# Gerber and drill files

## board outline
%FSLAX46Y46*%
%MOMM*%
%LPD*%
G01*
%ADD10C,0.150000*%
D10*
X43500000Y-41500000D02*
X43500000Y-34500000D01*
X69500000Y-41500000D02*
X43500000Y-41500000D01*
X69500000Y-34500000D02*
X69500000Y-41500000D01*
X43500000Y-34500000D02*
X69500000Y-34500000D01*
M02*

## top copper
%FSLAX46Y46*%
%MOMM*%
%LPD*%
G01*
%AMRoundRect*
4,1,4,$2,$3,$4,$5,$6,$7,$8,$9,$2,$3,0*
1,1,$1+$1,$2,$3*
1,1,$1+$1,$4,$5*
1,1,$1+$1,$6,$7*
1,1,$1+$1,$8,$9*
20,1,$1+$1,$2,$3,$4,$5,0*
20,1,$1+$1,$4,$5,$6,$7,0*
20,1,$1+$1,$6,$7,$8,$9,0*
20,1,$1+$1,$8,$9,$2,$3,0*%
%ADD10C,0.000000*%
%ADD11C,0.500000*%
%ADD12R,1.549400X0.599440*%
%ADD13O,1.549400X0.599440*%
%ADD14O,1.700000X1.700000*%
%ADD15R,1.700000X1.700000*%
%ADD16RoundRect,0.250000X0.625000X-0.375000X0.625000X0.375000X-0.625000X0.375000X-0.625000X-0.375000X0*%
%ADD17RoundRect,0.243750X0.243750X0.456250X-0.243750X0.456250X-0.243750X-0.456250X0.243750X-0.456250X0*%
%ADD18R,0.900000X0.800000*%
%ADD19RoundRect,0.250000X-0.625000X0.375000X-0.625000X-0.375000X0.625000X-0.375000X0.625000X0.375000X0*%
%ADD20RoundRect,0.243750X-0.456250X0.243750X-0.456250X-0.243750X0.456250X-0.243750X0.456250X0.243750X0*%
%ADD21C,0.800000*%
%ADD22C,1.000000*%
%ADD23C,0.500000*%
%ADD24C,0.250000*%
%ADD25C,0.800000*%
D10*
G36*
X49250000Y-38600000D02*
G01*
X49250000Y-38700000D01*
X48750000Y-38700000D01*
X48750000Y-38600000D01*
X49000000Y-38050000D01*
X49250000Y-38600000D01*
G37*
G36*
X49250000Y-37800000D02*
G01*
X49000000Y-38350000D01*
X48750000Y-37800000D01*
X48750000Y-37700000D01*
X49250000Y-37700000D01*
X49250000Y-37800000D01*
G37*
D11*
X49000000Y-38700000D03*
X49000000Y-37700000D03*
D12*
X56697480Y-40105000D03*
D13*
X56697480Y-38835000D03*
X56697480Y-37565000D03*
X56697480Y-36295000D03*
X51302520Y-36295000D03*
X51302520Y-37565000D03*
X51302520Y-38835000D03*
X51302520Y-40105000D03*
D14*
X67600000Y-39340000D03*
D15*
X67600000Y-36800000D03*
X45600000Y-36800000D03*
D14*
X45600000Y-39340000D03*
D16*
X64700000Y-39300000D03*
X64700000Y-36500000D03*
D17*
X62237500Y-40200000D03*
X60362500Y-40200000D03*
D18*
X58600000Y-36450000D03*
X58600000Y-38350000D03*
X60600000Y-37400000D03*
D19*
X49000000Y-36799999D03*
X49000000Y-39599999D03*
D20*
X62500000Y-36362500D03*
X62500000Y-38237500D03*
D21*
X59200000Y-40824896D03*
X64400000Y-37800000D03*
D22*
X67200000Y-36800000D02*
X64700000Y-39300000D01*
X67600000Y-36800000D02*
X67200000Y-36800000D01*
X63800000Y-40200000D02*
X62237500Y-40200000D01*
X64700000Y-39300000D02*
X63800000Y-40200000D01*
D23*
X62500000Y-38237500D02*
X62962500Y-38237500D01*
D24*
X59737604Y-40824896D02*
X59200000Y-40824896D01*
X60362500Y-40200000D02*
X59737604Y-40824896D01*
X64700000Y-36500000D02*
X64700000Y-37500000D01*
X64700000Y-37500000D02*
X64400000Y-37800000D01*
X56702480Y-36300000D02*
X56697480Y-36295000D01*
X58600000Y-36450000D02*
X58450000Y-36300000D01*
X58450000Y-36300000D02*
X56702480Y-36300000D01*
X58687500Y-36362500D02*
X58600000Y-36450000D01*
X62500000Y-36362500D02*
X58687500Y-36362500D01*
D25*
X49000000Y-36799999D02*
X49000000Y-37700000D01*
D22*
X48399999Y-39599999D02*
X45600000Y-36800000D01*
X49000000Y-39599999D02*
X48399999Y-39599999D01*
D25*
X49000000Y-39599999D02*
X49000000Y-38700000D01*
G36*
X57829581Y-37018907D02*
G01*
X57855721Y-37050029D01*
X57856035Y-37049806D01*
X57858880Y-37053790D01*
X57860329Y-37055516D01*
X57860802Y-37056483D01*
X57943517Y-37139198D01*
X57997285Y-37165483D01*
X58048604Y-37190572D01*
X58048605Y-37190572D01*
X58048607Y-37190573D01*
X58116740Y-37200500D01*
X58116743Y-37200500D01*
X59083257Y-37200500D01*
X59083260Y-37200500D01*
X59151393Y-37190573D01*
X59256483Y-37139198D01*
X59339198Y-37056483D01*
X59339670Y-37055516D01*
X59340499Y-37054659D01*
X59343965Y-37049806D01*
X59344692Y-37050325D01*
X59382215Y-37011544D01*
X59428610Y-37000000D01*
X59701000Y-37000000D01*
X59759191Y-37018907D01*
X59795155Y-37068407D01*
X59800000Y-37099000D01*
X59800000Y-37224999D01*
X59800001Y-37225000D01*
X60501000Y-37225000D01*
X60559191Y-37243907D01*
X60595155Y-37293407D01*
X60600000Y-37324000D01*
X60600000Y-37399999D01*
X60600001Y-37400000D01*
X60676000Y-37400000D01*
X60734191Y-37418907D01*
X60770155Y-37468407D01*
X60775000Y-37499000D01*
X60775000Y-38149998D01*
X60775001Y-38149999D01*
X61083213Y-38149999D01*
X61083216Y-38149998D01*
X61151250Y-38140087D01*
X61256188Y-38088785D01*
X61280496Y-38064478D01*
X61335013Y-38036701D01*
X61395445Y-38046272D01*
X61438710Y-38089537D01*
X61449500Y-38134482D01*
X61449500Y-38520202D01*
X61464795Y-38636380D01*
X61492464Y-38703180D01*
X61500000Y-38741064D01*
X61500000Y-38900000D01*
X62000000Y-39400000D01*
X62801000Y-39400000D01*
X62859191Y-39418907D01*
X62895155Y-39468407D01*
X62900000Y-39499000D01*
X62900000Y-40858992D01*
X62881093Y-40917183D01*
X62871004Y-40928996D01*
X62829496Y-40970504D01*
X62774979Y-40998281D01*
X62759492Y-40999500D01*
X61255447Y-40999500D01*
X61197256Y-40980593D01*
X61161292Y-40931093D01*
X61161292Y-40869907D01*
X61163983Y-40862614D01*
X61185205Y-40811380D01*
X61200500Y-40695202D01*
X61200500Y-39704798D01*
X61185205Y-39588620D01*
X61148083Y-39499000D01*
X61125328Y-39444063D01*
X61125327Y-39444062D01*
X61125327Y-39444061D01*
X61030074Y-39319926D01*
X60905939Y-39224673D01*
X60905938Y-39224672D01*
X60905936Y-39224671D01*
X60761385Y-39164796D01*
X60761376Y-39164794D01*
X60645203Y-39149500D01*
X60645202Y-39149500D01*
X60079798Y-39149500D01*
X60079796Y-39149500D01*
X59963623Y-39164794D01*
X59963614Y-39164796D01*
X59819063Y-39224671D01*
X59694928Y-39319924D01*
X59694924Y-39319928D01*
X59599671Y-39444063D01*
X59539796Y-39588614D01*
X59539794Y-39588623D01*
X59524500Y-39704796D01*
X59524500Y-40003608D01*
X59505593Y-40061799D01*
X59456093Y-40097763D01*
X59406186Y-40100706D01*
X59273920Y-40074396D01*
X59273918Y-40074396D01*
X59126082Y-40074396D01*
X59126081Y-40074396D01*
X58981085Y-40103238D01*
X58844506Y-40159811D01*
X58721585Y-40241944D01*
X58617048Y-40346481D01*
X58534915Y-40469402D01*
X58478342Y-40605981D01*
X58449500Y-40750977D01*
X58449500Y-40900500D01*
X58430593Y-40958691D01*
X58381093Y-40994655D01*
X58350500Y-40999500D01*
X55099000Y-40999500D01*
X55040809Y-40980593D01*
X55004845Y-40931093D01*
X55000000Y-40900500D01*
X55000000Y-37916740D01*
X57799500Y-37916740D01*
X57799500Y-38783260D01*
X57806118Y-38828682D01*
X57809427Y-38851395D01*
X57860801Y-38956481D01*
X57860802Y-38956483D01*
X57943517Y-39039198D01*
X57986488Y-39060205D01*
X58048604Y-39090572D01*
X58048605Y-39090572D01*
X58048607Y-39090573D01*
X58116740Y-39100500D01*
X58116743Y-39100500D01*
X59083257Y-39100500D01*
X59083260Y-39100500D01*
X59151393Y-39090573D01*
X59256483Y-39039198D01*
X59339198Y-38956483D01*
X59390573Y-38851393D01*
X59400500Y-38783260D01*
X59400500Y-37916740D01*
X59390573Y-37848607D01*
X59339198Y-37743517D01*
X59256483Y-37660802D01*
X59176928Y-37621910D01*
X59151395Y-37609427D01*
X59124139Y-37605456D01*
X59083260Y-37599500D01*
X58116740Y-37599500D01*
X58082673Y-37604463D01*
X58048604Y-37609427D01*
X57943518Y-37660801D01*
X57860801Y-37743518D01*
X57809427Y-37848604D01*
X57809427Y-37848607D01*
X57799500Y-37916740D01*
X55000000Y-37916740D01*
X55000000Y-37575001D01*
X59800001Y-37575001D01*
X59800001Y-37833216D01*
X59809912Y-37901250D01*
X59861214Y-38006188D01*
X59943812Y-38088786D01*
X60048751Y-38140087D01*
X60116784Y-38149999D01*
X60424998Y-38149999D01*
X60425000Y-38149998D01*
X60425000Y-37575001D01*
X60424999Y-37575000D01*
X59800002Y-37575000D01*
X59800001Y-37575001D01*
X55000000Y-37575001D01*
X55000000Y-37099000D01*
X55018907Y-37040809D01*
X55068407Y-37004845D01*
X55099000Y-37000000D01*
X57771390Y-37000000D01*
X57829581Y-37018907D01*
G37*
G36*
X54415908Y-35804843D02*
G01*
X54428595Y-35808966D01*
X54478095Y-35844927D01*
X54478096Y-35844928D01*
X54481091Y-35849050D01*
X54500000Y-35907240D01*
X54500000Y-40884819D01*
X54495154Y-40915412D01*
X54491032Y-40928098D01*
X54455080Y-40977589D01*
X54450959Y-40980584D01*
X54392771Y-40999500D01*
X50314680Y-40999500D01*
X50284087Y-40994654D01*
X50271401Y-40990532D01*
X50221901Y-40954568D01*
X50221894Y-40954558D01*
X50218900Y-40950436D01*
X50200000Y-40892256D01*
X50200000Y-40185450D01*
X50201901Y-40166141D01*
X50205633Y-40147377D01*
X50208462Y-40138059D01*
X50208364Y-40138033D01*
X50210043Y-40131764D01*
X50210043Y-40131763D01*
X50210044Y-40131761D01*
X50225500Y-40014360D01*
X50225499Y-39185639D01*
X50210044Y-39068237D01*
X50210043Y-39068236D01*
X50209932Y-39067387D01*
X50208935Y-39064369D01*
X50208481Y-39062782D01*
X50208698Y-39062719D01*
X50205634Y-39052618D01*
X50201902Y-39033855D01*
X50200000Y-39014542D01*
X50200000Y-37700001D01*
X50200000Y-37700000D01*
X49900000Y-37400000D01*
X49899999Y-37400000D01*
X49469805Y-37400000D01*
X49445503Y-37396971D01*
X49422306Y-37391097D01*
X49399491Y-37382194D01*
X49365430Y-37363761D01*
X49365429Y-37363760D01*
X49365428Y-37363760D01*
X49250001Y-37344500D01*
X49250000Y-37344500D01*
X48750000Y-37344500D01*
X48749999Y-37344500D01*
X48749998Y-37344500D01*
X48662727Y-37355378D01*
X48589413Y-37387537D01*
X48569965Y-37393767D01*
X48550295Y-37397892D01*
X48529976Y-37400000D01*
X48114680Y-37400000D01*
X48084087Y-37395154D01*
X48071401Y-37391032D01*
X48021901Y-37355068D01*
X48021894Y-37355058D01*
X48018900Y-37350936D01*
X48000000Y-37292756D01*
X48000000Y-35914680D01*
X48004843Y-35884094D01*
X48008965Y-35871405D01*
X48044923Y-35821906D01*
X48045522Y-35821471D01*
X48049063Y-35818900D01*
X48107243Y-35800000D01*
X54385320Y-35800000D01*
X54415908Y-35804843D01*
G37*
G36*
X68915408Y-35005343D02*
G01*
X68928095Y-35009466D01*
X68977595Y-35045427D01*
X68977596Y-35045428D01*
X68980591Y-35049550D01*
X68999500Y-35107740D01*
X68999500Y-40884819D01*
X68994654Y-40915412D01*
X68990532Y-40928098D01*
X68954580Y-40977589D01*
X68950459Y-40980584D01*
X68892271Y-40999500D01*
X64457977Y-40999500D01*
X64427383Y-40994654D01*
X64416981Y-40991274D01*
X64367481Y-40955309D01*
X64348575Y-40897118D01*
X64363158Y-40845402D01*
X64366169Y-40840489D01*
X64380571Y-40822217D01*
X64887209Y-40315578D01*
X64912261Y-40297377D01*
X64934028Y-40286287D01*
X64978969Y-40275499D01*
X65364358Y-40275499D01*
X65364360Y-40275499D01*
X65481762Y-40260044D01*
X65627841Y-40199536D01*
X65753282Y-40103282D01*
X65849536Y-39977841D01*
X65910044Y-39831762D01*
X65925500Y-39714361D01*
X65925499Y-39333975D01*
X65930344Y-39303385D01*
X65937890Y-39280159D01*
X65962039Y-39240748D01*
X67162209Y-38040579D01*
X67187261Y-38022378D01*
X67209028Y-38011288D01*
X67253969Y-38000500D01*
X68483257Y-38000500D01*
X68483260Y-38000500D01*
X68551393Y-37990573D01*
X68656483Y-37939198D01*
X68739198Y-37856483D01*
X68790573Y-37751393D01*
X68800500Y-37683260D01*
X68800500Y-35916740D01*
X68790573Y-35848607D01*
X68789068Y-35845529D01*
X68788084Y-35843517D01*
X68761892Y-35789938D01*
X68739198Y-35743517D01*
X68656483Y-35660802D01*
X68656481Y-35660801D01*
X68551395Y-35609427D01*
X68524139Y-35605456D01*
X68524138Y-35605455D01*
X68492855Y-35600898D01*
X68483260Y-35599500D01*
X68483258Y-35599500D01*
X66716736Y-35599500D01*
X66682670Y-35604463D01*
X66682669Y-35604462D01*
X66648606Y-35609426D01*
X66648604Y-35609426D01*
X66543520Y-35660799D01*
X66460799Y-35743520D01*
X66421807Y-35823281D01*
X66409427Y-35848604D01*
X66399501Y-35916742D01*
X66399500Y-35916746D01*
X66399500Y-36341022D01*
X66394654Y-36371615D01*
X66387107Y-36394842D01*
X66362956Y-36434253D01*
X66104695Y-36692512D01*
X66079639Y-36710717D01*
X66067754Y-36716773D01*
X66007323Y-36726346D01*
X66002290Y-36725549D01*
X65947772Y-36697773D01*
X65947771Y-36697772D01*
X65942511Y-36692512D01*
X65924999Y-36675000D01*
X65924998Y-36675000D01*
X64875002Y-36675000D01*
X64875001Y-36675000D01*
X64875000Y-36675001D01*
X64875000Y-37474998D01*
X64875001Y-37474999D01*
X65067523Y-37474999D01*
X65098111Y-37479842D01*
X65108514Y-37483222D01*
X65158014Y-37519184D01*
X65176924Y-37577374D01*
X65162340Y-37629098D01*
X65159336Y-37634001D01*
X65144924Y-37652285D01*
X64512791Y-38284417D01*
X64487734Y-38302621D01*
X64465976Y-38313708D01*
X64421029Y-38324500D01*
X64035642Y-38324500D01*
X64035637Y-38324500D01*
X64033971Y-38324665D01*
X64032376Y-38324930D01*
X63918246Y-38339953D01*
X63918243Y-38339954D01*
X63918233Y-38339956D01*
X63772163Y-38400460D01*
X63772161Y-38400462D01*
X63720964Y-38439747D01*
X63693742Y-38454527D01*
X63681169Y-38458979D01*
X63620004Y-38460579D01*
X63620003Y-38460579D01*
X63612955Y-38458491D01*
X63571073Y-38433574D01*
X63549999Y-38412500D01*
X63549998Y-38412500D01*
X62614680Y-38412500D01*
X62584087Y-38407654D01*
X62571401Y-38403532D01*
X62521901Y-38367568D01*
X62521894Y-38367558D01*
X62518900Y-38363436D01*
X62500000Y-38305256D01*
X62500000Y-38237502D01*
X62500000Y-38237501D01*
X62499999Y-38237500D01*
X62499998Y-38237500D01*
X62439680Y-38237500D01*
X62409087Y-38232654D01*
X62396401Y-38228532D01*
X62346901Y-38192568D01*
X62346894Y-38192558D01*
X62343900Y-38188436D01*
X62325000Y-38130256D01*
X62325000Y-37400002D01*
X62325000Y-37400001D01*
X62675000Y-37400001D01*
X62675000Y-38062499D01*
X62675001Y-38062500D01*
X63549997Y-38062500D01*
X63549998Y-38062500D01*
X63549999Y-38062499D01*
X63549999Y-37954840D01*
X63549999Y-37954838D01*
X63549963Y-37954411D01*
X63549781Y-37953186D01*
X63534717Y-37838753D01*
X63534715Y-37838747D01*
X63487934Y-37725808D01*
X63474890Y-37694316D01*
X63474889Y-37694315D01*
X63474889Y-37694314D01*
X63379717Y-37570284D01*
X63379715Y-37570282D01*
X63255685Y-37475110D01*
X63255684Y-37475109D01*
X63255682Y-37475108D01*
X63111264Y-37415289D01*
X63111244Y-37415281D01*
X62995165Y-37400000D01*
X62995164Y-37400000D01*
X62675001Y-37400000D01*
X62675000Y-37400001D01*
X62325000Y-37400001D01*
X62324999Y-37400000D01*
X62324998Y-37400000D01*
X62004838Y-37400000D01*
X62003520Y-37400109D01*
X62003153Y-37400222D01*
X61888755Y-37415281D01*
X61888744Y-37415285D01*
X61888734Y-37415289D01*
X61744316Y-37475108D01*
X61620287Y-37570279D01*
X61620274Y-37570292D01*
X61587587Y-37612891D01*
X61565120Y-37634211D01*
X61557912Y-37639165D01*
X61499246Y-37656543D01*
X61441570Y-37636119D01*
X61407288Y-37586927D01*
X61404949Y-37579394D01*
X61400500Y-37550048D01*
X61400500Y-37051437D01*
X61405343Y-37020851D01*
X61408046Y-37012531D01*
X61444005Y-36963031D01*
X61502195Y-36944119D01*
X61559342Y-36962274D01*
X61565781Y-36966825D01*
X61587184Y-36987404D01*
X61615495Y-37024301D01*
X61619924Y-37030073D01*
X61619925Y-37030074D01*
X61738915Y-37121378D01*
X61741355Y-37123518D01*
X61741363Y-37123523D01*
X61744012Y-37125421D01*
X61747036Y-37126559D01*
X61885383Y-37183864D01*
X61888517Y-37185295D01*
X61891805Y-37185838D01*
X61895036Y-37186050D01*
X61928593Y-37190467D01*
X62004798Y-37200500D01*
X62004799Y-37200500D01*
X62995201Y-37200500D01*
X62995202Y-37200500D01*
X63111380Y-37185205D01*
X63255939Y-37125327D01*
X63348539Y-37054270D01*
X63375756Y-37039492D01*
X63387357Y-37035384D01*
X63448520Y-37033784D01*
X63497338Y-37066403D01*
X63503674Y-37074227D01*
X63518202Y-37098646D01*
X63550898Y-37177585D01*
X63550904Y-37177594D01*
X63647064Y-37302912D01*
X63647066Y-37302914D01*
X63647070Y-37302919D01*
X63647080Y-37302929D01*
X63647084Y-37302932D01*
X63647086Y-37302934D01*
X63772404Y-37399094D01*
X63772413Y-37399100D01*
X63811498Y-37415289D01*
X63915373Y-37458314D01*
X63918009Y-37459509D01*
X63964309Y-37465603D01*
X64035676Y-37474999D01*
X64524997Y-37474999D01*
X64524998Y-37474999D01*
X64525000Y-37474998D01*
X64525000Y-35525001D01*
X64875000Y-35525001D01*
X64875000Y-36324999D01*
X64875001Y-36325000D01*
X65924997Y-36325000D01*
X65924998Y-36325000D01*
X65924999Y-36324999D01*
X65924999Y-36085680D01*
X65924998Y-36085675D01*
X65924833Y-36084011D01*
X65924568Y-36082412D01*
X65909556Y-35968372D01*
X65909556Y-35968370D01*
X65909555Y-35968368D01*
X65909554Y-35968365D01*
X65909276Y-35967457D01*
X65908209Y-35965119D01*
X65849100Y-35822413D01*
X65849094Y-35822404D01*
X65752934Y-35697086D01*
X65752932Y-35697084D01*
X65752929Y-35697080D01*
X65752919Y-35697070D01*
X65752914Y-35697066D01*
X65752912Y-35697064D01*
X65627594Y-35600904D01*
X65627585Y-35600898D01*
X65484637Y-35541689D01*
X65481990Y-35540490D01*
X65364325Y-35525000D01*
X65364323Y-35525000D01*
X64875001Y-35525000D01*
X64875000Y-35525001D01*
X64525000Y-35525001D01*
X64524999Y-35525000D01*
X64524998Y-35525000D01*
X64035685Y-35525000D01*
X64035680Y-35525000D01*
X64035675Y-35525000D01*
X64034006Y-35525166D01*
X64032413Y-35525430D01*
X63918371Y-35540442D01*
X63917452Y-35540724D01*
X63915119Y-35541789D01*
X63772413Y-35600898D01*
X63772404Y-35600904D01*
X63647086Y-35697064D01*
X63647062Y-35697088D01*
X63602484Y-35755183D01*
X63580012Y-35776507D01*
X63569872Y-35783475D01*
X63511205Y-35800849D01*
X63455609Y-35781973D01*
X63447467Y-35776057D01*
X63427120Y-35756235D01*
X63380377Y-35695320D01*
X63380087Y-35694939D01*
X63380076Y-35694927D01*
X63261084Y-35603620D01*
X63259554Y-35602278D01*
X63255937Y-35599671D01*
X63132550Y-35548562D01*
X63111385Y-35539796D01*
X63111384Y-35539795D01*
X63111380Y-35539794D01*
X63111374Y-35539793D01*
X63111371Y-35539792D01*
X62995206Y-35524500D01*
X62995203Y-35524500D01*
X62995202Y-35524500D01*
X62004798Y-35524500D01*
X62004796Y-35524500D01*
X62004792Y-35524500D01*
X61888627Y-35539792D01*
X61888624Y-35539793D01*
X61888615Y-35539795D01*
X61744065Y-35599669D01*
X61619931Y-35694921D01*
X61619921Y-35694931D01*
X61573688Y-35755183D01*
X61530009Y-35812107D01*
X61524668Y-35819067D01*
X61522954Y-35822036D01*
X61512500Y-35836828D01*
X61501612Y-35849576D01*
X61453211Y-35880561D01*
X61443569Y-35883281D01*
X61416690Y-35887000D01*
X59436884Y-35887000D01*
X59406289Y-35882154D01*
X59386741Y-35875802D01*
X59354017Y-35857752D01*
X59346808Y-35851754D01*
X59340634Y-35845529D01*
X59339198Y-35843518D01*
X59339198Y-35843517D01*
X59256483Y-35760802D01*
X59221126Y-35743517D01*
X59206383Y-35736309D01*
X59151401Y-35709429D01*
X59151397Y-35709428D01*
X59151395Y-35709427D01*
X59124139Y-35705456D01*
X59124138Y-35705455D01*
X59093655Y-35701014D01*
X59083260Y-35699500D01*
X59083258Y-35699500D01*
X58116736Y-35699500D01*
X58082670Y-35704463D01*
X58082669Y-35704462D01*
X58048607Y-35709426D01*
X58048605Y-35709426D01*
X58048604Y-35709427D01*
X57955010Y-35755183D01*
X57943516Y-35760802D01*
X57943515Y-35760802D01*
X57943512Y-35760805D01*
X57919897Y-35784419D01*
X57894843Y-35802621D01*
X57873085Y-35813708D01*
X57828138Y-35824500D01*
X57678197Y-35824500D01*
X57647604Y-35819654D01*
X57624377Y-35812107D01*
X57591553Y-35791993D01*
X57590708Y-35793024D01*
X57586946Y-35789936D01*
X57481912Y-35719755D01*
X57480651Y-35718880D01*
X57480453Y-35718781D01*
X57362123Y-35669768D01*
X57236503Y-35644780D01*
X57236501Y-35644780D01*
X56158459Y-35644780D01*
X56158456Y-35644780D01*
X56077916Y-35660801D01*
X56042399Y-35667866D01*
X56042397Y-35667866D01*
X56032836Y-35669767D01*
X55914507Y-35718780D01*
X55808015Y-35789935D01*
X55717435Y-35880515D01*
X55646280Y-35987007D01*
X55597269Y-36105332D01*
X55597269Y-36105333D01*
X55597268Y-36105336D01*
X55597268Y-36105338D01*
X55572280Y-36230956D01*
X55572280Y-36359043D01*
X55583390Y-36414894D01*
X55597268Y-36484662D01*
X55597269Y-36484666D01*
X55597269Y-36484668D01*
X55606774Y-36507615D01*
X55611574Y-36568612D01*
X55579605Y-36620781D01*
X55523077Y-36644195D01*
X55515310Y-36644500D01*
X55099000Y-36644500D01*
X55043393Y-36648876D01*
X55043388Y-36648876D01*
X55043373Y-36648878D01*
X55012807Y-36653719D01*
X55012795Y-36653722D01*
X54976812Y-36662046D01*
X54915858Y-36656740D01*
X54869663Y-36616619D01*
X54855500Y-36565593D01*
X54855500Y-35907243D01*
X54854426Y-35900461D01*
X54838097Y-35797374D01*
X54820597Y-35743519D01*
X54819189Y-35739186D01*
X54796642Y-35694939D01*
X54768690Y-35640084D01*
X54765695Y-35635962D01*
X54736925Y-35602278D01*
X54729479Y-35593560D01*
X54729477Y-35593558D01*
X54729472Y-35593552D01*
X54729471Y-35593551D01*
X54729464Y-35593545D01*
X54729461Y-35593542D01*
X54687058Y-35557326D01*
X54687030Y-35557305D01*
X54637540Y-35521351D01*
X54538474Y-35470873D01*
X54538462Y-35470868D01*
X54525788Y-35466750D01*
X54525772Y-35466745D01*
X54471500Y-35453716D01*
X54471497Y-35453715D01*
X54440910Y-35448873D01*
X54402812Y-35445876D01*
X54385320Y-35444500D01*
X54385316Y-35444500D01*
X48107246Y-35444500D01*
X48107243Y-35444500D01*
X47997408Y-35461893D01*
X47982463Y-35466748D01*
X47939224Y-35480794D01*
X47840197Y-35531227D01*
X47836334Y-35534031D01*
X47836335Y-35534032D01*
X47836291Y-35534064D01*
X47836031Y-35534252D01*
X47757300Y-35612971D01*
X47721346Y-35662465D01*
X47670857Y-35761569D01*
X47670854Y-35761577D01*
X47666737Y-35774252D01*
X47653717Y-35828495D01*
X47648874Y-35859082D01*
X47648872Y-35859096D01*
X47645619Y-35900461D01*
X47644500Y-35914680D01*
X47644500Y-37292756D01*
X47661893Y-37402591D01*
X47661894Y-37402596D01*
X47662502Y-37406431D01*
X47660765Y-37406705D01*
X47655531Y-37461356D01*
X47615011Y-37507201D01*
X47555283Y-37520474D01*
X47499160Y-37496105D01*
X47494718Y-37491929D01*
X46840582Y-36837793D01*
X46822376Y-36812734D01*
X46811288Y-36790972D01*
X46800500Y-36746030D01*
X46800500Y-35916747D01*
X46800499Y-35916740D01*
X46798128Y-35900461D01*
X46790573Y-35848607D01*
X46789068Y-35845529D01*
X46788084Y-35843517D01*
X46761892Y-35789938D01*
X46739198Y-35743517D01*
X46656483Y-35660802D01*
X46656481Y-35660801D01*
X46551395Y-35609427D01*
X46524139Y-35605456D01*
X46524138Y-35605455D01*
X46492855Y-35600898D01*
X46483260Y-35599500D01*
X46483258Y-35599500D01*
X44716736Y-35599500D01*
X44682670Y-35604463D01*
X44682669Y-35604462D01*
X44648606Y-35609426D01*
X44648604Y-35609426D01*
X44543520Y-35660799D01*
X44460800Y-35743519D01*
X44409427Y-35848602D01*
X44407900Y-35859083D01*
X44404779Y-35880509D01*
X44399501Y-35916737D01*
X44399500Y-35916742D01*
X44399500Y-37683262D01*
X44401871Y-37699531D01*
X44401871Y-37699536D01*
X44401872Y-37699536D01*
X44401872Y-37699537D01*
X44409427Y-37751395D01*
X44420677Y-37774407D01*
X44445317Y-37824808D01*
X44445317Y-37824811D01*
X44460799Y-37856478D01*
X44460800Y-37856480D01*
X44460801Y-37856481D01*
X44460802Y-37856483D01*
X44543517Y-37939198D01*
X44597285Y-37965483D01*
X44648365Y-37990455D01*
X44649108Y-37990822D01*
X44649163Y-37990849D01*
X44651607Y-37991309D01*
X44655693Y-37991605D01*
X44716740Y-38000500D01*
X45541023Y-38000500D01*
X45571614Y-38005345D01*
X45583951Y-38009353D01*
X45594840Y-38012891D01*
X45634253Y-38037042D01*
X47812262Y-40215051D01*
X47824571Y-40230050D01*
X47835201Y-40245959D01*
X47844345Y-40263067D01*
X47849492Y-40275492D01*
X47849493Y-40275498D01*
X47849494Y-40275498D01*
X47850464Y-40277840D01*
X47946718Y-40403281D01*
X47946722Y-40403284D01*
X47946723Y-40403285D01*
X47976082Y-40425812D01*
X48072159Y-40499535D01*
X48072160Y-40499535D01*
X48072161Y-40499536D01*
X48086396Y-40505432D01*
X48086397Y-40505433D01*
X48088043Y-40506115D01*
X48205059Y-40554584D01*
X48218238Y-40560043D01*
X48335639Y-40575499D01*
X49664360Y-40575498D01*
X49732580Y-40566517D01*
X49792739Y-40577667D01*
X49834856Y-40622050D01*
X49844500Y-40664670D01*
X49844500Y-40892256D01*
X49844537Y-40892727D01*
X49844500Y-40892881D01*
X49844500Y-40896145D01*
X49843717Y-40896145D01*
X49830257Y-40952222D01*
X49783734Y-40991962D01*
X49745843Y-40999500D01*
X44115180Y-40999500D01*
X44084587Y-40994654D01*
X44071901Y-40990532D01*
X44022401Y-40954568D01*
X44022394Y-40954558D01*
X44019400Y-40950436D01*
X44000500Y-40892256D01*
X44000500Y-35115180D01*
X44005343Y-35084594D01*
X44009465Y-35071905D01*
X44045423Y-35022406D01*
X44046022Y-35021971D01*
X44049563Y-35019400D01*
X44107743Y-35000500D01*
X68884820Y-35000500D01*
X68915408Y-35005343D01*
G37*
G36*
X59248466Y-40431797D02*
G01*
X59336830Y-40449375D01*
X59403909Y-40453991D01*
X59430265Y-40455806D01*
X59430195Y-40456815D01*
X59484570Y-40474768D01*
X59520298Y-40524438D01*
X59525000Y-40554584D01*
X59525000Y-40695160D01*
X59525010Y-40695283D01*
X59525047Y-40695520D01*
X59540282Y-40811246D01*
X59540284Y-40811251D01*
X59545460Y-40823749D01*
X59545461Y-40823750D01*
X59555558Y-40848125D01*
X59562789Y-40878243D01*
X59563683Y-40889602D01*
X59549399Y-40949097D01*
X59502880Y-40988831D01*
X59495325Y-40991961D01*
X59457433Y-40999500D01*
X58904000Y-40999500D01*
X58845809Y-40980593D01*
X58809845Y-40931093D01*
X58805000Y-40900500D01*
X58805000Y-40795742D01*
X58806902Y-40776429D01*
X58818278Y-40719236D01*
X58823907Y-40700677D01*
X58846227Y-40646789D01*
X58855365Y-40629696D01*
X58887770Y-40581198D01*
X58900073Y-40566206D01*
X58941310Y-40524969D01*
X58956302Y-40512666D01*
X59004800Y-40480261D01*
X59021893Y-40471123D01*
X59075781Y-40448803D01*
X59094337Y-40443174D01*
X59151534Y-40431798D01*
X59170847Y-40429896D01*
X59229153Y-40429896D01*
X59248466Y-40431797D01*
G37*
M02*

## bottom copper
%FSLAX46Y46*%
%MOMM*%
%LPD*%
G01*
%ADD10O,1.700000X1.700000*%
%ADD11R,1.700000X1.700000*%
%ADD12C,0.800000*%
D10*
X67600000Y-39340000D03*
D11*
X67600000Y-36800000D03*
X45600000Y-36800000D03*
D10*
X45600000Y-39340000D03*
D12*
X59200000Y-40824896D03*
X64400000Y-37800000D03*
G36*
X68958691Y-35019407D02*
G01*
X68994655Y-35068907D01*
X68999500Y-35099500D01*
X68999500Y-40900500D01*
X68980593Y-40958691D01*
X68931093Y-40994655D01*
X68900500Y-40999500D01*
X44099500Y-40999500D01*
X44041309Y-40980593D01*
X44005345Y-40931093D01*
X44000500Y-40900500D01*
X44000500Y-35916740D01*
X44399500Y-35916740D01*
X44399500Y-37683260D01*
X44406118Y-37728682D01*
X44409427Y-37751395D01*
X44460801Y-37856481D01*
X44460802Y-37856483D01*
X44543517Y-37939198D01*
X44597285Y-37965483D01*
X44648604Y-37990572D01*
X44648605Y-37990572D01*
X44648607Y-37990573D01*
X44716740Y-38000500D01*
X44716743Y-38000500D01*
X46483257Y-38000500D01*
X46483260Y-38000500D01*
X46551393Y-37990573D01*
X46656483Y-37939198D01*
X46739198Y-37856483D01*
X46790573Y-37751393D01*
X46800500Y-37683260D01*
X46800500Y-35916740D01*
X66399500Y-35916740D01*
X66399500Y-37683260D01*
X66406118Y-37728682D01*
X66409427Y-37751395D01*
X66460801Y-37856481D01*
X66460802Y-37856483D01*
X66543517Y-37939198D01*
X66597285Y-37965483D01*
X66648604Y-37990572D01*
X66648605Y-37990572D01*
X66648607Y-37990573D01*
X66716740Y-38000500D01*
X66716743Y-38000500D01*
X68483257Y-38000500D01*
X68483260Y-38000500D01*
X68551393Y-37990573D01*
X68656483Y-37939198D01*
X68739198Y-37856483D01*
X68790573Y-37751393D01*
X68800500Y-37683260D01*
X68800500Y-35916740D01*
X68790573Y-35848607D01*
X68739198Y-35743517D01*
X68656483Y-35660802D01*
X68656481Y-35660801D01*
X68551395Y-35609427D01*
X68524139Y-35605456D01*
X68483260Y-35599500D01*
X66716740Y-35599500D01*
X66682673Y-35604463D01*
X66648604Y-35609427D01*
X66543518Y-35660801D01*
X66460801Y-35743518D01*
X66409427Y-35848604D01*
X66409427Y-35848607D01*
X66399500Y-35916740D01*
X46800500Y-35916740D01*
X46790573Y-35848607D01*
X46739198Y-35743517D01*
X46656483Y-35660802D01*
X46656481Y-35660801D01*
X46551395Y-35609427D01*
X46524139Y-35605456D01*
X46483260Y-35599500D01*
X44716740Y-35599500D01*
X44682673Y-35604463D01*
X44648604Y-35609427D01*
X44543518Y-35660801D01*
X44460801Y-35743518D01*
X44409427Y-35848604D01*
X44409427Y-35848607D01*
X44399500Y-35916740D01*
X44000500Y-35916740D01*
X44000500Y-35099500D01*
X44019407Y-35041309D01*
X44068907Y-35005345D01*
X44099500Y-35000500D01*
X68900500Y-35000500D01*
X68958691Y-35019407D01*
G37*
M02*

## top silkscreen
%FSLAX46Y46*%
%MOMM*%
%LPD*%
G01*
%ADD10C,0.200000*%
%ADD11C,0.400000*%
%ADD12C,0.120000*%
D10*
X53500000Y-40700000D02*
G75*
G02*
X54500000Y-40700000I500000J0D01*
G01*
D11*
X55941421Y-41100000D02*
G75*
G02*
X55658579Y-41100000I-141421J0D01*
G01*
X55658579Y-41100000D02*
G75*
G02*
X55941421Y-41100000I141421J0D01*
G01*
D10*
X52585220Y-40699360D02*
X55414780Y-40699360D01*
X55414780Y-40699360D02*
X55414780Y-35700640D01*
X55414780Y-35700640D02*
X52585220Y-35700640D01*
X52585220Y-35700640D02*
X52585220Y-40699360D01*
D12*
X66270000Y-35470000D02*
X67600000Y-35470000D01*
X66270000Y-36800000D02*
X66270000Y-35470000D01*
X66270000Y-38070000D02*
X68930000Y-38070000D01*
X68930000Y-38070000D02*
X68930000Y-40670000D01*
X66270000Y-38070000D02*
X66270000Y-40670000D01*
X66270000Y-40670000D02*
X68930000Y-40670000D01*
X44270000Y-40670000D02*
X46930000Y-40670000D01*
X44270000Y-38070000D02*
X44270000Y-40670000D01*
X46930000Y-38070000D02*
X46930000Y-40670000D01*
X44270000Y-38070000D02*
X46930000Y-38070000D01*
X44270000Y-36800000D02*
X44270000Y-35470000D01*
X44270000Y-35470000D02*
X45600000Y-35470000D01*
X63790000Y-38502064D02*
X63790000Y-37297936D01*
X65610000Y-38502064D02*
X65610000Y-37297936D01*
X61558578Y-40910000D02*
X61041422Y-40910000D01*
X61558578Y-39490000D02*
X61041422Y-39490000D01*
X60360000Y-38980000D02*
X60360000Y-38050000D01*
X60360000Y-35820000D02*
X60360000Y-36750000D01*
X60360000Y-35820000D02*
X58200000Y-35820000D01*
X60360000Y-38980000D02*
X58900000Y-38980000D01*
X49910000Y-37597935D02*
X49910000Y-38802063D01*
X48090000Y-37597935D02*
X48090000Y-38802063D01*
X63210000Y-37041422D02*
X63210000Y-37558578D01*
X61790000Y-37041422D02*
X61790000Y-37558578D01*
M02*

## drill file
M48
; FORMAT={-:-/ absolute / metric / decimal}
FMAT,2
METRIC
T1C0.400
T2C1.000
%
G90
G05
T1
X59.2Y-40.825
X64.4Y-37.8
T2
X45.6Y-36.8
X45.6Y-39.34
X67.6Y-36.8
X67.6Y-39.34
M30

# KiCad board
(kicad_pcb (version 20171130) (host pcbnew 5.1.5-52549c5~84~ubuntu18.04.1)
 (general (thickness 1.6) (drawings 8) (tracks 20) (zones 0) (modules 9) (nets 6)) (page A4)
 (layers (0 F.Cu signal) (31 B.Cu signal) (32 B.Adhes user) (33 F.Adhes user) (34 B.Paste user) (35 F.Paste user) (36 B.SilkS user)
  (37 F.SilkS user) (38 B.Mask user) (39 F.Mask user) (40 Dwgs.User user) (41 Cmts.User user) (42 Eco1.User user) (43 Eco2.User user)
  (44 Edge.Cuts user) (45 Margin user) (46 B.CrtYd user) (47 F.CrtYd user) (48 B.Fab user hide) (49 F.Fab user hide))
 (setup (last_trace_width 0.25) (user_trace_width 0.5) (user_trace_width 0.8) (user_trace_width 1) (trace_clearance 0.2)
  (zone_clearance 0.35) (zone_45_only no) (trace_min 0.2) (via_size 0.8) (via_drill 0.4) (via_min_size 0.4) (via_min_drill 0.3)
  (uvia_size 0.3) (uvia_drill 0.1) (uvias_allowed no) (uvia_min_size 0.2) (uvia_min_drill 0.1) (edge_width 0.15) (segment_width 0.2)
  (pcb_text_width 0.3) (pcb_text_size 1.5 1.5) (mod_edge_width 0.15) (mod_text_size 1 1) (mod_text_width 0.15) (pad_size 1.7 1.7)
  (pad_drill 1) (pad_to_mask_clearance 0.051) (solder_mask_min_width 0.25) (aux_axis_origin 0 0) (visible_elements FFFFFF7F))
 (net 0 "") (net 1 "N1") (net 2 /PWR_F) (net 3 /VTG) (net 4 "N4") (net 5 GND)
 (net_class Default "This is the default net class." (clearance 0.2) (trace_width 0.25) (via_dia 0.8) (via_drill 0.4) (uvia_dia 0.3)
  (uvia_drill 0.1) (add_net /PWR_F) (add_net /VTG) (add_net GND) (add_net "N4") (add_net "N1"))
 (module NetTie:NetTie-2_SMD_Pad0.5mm (layer F.Cu) (at 49 38.2 90)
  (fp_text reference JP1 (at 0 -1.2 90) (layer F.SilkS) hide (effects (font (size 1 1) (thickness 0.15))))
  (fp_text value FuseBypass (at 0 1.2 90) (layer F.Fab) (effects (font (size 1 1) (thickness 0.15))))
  (fp_poly (pts (xy -0.5 -0.25) (xy -0.4 -0.25) (xy 0.15 0) (xy -0.4 0.25) (xy -0.5 0.25)) (layer F.Cu) (width 0))
  (fp_poly (pts (xy 0.5 0.25) (xy 0.4 0.25) (xy -0.15 0) (xy 0.4 -0.25) (xy 0.5 -0.25)) (layer F.Cu) (width 0))
  (pad 1 smd circle (at -0.5 0 90) (size 0.5 0.5) (layers F.Cu) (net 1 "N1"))
  (pad 2 smd circle (at 0.5 0 90) (size 0.5 0.5) (layers F.Cu) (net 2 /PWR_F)))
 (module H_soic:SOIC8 (layer F.Cu) (at 54 38.2 180)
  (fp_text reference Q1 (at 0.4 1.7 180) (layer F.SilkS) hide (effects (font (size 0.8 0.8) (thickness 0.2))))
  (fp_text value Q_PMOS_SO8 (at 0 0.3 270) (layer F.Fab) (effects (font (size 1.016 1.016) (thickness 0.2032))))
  (fp_arc (start 0 -2.5) (end 0.5 -2.5) (angle 180) (layer F.SilkS) (width 0.2))
  (fp_circle (center -1.8 -2.9) (end -1.7 -2.8) (layer F.SilkS) (width 0.4))
  (fp_line (start 1.41478 -2.49936) (end -1.41478 -2.49936) (layer F.SilkS) (width 0.2))
  (fp_line (start -1.41478 -2.49936) (end -1.41478 2.49936) (layer F.SilkS) (width 0.2))
  (fp_line (start -1.41478 2.49936) (end 1.41478 2.49936) (layer F.SilkS) (width 0.2))
  (fp_line (start 1.41478 2.49936) (end 1.41478 -2.49936) (layer F.SilkS) (width 0.2))
  (pad 1 smd rect (at -2.69748 -1.905 180) (size 1.5494 0.59944) (layers F.Cu F.Paste F.Mask) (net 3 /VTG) (zone_connect 2))
  (pad 2 smd oval (at -2.69748 -0.635 180) (size 1.5494 0.59944) (layers F.Cu F.Paste F.Mask) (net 3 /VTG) (zone_connect 2))
  (pad 3 smd oval (at -2.69748 0.635 180) (size 1.5494 0.59944) (layers F.Cu F.Paste F.Mask) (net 3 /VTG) (zone_connect 2))
  (pad 4 smd oval (at -2.69748 1.905 180) (size 1.5494 0.59944) (layers F.Cu F.Paste F.Mask) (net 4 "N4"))
  (pad 5 smd oval (at 2.69748 1.905 180) (size 1.5494 0.59944) (layers F.Cu F.Paste F.Mask) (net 2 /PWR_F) (zone_connect 2))
  (pad 6 smd oval (at 2.69748 0.635 180) (size 1.5494 0.59944) (layers F.Cu F.Paste F.Mask) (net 2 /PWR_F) (zone_connect 2))
  (pad 7 smd oval (at 2.69748 -0.635 180) (size 1.5494 0.59944) (layers F.Cu F.Paste F.Mask) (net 2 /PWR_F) (zone_connect 2))
  (pad 8 smd oval (at 2.69748 -1.905 180) (size 1.5494 0.59944) (layers F.Cu F.Paste F.Mask) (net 2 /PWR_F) (zone_connect 2)))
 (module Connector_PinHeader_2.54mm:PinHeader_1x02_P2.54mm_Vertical (layer F.Cu) (at 67.6 36.8)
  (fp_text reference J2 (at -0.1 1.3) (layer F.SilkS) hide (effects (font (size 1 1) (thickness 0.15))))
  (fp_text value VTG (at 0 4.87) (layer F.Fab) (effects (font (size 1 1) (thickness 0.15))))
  (fp_line (start -1.33 -1.33) (end 0 -1.33) (layer F.SilkS) (width 0.12))
  (fp_line (start -1.33 0) (end -1.33 -1.33) (layer F.SilkS) (width 0.12))
  (fp_line (start -1.33 1.27) (end 1.33 1.27) (layer F.SilkS) (width 0.12))
  (fp_line (start 1.33 1.27) (end 1.33 3.87) (layer F.SilkS) (width 0.12))
  (fp_line (start -1.33 1.27) (end -1.33 3.87) (layer F.SilkS) (width 0.12))
  (fp_line (start -1.33 3.87) (end 1.33 3.87) (layer F.SilkS) (width 0.12))
  (pad 2 thru_hole oval (at 0 2.54) (size 1.7 1.7) (drill 1) (layers *.Cu *.Mask) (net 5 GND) (zone_connect 2))
  (pad 1 thru_hole rect (at 0 0) (size 1.7 1.7) (drill 1) (layers *.Cu *.Mask) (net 3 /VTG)))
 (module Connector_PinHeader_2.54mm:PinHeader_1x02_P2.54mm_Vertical (layer F.Cu) (at 45.6 36.8)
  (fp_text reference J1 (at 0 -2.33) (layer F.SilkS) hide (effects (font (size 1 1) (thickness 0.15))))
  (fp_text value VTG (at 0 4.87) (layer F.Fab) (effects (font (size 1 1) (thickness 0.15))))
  (fp_line (start -1.33 3.87) (end 1.33 3.87) (layer F.SilkS) (width 0.12))
  (fp_line (start -1.33 1.27) (end -1.33 3.87) (layer F.SilkS) (width 0.12))
  (fp_line (start 1.33 1.27) (end 1.33 3.87) (layer F.SilkS) (width 0.12))
  (fp_line (start -1.33 1.27) (end 1.33 1.27) (layer F.SilkS) (width 0.12))
  (fp_line (start -1.33 0) (end -1.33 -1.33) (layer F.SilkS) (width 0.12))
  (fp_line (start -1.33 -1.33) (end 0 -1.33) (layer F.SilkS) (width 0.12))
  (pad 1 thru_hole rect (at 0 0) (size 1.7 1.7) (drill 1) (layers *.Cu *.Mask) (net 1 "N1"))
  (pad 2 thru_hole oval (at 0 2.54) (size 1.7 1.7) (drill 1) (layers *.Cu *.Mask) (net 5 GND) (zone_connect 2)))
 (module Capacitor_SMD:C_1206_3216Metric (layer F.Cu) (at 64.7 37.9 90)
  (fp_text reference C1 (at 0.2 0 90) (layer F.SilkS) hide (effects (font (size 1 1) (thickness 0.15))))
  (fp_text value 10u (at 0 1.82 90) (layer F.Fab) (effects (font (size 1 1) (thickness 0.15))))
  (fp_line (start -0.602064 -0.91) (end 0.602064 -0.91) (layer F.SilkS) (width 0.12))
  (fp_line (start -0.602064 0.91) (end 0.602064 0.91) (layer F.SilkS) (width 0.12))
  (pad 1 smd roundrect (at -1.4 0 90) (size 1.25 1.75) (layers F.Cu F.Paste F.Mask) (roundrect_rratio 0.2) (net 3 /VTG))
  (pad 2 smd roundrect (at 1.4 0 90) (size 1.25 1.75) (layers F.Cu F.Paste F.Mask) (roundrect_rratio 0.2) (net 5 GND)))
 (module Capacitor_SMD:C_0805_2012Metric (layer F.Cu) (at 61.3 40.2 180)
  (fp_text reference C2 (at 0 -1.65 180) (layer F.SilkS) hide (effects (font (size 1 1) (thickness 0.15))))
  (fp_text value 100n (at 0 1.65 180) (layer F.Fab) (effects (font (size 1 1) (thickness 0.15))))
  (fp_line (start -0.258578 -0.71) (end 0.258578 -0.71) (layer F.SilkS) (width 0.12))
  (fp_line (start -0.258578 0.71) (end 0.258578 0.71) (layer F.SilkS) (width 0.12))
  (pad 1 smd roundrect (at -0.9375 0 180) (size 0.975 1.4) (layers F.Cu F.Paste F.Mask) (roundrect_rratio 0.25) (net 3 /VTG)
   (zone_connect 2))
  (pad 2 smd roundrect (at 0.9375 0 180) (size 0.975 1.4) (layers F.Cu F.Paste F.Mask) (roundrect_rratio 0.25) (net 5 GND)))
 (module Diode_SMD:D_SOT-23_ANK (layer F.Cu) (at 59.6 37.4)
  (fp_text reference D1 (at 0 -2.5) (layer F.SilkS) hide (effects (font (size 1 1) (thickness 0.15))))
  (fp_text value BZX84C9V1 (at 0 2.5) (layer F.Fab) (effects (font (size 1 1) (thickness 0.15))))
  (fp_line (start 0.76 1.58) (end 0.76 0.65) (layer F.SilkS) (width 0.12))
  (fp_line (start 0.76 -1.58) (end 0.76 -0.65) (layer F.SilkS) (width 0.12))
  (fp_line (start 0.76 -1.58) (end -1.4 -1.58) (layer F.SilkS) (width 0.12))
  (fp_line (start 0.76 1.58) (end -0.7 1.58) (layer F.SilkS) (width 0.12))
  (pad 2 smd rect (at -1 -0.95) (size 0.9 0.8) (layers F.Cu F.Paste F.Mask) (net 4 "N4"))
  (pad "" smd rect (at -1 0.95) (size 0.9 0.8) (layers F.Cu F.Paste F.Mask))
  (pad 1 smd rect (at 1 0) (size 0.9 0.8) (layers F.Cu F.Paste F.Mask) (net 3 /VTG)))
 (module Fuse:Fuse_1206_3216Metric (layer F.Cu) (at 49 38.199999 270)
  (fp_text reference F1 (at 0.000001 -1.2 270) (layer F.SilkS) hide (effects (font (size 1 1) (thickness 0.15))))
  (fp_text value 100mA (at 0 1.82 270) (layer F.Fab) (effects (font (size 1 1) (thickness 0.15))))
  (fp_line (start -0.602064 -0.91) (end 0.602064 -0.91) (layer F.SilkS) (width 0.12))
  (fp_line (start -0.602064 0.91) (end 0.602064 0.91) (layer F.SilkS) (width 0.12))
  (pad 1 smd roundrect (at -1.4 0 270) (size 1.25 1.75) (layers F.Cu F.Paste F.Mask) (roundrect_rratio 0.2) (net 2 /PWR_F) (zone_connect 2))
  (pad 2 smd roundrect (at 1.4 0 270) (size 1.25 1.75) (layers F.Cu F.Paste F.Mask) (roundrect_rratio 0.2) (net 1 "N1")))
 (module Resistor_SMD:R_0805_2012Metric (layer F.Cu) (at 62.5 37.3 270)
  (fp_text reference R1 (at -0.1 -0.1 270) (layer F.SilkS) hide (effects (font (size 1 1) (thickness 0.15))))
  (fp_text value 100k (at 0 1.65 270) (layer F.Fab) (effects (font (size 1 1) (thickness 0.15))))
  (fp_line (start -0.258578 -0.71) (end 0.258578 -0.71) (layer F.SilkS) (width 0.12))
  (fp_line (start -0.258578 0.71) (end 0.258578 0.71) (layer F.SilkS) (width 0.12))
  (pad 1 smd roundrect (at -0.9375 0 270) (size 0.975 1.4) (layers F.Cu F.Paste F.Mask) (roundrect_rratio 0.25) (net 4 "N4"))
  (pad 2 smd roundrect (at 0.9375 0 270) (size 0.975 1.4) (layers F.Cu F.Paste F.Mask) (roundrect_rratio 0.25) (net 5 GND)))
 (gr_line (start 43.5 41.5) (end 43.5 34.5) (layer Edge.Cuts) (width 0.15))
 (gr_line (start 69.5 41.5) (end 43.5 41.5) (layer Edge.Cuts) (width 0.15))
 (gr_line (start 69.5 34.5) (end 69.5 41.5) (layer Edge.Cuts) (width 0.15))
 (gr_line (start 43.5 34.5) (end 69.5 34.5) (layer Edge.Cuts) (width 0.15))
 (segment (start 67.2 36.8) (end 64.7 39.3) (width 1) (layer F.Cu) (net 3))
 (segment (start 67.6 36.8) (end 67.2 36.8) (width 1) (layer F.Cu) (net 3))
 (segment (start 63.8 40.2) (end 62.2375 40.2) (width 1) (layer F.Cu) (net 3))
 (segment (start 64.7 39.3) (end 63.8 40.2) (width 1) (layer F.Cu) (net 3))
 (segment (start 62.5 38.2375) (end 62.9625 38.2375) (width 0.5) (layer F.Cu) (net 5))
 (via (at 59.2 40.824896) (size 0.8) (drill 0.4) (layers F.Cu B.Cu) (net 5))
 (segment (start 59.737604 40.824896) (end 59.2 40.824896) (width 0.25) (layer F.Cu) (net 5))
 (segment (start 60.3625 40.2) (end 59.737604 40.824896) (width 0.25) (layer F.Cu) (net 5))
 (via (at 64.4 37.8) (size 0.8) (drill 0.4) (layers F.Cu B.Cu) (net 5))
 (segment (start 64.7 36.5) (end 64.7 37.5) (width 0.25) (layer F.Cu) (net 5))
 (segment (start 64.7 37.5) (end 64.4 37.8) (width 0.25) (layer F.Cu) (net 5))
 (segment (start 56.70248 36.3) (end 56.69748 36.295) (width 0.25) (layer F.Cu) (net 4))
 (segment (start 58.6 36.45) (end 58.45 36.3) (width 0.25) (layer F.Cu) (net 4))
 (segment (start 58.45 36.3) (end 56.70248 36.3) (width 0.25) (layer F.Cu) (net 4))
 (segment (start 58.6875 36.3625) (end 58.6 36.45) (width 0.25) (layer F.Cu) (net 4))
 (segment (start 62.5 36.3625) (end 58.6875 36.3625) (width 0.25) (layer F.Cu) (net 4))
 (segment (start 49 36.799999) (end 49 37.7) (width 0.8) (layer F.Cu) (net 2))
 (segment (start 48.399999 39.599999) (end 45.6 36.8) (width 1) (layer F.Cu) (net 1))
 (segment (start 49 39.599999) (end 48.399999 39.599999) (width 1) (layer F.Cu) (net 1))
 (segment (start 49 39.599999) (end 49 38.7) (width 0.8) (layer F.Cu) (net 1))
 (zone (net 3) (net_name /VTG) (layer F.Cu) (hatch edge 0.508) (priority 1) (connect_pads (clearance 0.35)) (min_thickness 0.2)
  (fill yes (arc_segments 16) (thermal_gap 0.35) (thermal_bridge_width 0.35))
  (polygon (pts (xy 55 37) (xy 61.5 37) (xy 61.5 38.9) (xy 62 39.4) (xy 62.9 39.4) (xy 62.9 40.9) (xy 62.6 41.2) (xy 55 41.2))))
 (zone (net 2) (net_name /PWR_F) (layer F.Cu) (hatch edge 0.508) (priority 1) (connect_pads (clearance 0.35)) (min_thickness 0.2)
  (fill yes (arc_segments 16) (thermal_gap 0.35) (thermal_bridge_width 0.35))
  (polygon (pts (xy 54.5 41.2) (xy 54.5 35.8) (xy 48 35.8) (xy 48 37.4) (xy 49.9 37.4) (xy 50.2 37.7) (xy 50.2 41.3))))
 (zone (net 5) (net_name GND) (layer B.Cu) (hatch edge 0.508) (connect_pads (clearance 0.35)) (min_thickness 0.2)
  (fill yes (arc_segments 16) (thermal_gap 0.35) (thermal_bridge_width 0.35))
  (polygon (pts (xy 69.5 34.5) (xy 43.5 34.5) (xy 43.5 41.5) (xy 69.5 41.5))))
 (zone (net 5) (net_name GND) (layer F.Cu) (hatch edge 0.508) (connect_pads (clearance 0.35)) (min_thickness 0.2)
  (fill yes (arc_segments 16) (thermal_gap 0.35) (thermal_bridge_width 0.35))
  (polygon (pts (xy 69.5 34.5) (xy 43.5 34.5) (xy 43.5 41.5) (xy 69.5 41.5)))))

